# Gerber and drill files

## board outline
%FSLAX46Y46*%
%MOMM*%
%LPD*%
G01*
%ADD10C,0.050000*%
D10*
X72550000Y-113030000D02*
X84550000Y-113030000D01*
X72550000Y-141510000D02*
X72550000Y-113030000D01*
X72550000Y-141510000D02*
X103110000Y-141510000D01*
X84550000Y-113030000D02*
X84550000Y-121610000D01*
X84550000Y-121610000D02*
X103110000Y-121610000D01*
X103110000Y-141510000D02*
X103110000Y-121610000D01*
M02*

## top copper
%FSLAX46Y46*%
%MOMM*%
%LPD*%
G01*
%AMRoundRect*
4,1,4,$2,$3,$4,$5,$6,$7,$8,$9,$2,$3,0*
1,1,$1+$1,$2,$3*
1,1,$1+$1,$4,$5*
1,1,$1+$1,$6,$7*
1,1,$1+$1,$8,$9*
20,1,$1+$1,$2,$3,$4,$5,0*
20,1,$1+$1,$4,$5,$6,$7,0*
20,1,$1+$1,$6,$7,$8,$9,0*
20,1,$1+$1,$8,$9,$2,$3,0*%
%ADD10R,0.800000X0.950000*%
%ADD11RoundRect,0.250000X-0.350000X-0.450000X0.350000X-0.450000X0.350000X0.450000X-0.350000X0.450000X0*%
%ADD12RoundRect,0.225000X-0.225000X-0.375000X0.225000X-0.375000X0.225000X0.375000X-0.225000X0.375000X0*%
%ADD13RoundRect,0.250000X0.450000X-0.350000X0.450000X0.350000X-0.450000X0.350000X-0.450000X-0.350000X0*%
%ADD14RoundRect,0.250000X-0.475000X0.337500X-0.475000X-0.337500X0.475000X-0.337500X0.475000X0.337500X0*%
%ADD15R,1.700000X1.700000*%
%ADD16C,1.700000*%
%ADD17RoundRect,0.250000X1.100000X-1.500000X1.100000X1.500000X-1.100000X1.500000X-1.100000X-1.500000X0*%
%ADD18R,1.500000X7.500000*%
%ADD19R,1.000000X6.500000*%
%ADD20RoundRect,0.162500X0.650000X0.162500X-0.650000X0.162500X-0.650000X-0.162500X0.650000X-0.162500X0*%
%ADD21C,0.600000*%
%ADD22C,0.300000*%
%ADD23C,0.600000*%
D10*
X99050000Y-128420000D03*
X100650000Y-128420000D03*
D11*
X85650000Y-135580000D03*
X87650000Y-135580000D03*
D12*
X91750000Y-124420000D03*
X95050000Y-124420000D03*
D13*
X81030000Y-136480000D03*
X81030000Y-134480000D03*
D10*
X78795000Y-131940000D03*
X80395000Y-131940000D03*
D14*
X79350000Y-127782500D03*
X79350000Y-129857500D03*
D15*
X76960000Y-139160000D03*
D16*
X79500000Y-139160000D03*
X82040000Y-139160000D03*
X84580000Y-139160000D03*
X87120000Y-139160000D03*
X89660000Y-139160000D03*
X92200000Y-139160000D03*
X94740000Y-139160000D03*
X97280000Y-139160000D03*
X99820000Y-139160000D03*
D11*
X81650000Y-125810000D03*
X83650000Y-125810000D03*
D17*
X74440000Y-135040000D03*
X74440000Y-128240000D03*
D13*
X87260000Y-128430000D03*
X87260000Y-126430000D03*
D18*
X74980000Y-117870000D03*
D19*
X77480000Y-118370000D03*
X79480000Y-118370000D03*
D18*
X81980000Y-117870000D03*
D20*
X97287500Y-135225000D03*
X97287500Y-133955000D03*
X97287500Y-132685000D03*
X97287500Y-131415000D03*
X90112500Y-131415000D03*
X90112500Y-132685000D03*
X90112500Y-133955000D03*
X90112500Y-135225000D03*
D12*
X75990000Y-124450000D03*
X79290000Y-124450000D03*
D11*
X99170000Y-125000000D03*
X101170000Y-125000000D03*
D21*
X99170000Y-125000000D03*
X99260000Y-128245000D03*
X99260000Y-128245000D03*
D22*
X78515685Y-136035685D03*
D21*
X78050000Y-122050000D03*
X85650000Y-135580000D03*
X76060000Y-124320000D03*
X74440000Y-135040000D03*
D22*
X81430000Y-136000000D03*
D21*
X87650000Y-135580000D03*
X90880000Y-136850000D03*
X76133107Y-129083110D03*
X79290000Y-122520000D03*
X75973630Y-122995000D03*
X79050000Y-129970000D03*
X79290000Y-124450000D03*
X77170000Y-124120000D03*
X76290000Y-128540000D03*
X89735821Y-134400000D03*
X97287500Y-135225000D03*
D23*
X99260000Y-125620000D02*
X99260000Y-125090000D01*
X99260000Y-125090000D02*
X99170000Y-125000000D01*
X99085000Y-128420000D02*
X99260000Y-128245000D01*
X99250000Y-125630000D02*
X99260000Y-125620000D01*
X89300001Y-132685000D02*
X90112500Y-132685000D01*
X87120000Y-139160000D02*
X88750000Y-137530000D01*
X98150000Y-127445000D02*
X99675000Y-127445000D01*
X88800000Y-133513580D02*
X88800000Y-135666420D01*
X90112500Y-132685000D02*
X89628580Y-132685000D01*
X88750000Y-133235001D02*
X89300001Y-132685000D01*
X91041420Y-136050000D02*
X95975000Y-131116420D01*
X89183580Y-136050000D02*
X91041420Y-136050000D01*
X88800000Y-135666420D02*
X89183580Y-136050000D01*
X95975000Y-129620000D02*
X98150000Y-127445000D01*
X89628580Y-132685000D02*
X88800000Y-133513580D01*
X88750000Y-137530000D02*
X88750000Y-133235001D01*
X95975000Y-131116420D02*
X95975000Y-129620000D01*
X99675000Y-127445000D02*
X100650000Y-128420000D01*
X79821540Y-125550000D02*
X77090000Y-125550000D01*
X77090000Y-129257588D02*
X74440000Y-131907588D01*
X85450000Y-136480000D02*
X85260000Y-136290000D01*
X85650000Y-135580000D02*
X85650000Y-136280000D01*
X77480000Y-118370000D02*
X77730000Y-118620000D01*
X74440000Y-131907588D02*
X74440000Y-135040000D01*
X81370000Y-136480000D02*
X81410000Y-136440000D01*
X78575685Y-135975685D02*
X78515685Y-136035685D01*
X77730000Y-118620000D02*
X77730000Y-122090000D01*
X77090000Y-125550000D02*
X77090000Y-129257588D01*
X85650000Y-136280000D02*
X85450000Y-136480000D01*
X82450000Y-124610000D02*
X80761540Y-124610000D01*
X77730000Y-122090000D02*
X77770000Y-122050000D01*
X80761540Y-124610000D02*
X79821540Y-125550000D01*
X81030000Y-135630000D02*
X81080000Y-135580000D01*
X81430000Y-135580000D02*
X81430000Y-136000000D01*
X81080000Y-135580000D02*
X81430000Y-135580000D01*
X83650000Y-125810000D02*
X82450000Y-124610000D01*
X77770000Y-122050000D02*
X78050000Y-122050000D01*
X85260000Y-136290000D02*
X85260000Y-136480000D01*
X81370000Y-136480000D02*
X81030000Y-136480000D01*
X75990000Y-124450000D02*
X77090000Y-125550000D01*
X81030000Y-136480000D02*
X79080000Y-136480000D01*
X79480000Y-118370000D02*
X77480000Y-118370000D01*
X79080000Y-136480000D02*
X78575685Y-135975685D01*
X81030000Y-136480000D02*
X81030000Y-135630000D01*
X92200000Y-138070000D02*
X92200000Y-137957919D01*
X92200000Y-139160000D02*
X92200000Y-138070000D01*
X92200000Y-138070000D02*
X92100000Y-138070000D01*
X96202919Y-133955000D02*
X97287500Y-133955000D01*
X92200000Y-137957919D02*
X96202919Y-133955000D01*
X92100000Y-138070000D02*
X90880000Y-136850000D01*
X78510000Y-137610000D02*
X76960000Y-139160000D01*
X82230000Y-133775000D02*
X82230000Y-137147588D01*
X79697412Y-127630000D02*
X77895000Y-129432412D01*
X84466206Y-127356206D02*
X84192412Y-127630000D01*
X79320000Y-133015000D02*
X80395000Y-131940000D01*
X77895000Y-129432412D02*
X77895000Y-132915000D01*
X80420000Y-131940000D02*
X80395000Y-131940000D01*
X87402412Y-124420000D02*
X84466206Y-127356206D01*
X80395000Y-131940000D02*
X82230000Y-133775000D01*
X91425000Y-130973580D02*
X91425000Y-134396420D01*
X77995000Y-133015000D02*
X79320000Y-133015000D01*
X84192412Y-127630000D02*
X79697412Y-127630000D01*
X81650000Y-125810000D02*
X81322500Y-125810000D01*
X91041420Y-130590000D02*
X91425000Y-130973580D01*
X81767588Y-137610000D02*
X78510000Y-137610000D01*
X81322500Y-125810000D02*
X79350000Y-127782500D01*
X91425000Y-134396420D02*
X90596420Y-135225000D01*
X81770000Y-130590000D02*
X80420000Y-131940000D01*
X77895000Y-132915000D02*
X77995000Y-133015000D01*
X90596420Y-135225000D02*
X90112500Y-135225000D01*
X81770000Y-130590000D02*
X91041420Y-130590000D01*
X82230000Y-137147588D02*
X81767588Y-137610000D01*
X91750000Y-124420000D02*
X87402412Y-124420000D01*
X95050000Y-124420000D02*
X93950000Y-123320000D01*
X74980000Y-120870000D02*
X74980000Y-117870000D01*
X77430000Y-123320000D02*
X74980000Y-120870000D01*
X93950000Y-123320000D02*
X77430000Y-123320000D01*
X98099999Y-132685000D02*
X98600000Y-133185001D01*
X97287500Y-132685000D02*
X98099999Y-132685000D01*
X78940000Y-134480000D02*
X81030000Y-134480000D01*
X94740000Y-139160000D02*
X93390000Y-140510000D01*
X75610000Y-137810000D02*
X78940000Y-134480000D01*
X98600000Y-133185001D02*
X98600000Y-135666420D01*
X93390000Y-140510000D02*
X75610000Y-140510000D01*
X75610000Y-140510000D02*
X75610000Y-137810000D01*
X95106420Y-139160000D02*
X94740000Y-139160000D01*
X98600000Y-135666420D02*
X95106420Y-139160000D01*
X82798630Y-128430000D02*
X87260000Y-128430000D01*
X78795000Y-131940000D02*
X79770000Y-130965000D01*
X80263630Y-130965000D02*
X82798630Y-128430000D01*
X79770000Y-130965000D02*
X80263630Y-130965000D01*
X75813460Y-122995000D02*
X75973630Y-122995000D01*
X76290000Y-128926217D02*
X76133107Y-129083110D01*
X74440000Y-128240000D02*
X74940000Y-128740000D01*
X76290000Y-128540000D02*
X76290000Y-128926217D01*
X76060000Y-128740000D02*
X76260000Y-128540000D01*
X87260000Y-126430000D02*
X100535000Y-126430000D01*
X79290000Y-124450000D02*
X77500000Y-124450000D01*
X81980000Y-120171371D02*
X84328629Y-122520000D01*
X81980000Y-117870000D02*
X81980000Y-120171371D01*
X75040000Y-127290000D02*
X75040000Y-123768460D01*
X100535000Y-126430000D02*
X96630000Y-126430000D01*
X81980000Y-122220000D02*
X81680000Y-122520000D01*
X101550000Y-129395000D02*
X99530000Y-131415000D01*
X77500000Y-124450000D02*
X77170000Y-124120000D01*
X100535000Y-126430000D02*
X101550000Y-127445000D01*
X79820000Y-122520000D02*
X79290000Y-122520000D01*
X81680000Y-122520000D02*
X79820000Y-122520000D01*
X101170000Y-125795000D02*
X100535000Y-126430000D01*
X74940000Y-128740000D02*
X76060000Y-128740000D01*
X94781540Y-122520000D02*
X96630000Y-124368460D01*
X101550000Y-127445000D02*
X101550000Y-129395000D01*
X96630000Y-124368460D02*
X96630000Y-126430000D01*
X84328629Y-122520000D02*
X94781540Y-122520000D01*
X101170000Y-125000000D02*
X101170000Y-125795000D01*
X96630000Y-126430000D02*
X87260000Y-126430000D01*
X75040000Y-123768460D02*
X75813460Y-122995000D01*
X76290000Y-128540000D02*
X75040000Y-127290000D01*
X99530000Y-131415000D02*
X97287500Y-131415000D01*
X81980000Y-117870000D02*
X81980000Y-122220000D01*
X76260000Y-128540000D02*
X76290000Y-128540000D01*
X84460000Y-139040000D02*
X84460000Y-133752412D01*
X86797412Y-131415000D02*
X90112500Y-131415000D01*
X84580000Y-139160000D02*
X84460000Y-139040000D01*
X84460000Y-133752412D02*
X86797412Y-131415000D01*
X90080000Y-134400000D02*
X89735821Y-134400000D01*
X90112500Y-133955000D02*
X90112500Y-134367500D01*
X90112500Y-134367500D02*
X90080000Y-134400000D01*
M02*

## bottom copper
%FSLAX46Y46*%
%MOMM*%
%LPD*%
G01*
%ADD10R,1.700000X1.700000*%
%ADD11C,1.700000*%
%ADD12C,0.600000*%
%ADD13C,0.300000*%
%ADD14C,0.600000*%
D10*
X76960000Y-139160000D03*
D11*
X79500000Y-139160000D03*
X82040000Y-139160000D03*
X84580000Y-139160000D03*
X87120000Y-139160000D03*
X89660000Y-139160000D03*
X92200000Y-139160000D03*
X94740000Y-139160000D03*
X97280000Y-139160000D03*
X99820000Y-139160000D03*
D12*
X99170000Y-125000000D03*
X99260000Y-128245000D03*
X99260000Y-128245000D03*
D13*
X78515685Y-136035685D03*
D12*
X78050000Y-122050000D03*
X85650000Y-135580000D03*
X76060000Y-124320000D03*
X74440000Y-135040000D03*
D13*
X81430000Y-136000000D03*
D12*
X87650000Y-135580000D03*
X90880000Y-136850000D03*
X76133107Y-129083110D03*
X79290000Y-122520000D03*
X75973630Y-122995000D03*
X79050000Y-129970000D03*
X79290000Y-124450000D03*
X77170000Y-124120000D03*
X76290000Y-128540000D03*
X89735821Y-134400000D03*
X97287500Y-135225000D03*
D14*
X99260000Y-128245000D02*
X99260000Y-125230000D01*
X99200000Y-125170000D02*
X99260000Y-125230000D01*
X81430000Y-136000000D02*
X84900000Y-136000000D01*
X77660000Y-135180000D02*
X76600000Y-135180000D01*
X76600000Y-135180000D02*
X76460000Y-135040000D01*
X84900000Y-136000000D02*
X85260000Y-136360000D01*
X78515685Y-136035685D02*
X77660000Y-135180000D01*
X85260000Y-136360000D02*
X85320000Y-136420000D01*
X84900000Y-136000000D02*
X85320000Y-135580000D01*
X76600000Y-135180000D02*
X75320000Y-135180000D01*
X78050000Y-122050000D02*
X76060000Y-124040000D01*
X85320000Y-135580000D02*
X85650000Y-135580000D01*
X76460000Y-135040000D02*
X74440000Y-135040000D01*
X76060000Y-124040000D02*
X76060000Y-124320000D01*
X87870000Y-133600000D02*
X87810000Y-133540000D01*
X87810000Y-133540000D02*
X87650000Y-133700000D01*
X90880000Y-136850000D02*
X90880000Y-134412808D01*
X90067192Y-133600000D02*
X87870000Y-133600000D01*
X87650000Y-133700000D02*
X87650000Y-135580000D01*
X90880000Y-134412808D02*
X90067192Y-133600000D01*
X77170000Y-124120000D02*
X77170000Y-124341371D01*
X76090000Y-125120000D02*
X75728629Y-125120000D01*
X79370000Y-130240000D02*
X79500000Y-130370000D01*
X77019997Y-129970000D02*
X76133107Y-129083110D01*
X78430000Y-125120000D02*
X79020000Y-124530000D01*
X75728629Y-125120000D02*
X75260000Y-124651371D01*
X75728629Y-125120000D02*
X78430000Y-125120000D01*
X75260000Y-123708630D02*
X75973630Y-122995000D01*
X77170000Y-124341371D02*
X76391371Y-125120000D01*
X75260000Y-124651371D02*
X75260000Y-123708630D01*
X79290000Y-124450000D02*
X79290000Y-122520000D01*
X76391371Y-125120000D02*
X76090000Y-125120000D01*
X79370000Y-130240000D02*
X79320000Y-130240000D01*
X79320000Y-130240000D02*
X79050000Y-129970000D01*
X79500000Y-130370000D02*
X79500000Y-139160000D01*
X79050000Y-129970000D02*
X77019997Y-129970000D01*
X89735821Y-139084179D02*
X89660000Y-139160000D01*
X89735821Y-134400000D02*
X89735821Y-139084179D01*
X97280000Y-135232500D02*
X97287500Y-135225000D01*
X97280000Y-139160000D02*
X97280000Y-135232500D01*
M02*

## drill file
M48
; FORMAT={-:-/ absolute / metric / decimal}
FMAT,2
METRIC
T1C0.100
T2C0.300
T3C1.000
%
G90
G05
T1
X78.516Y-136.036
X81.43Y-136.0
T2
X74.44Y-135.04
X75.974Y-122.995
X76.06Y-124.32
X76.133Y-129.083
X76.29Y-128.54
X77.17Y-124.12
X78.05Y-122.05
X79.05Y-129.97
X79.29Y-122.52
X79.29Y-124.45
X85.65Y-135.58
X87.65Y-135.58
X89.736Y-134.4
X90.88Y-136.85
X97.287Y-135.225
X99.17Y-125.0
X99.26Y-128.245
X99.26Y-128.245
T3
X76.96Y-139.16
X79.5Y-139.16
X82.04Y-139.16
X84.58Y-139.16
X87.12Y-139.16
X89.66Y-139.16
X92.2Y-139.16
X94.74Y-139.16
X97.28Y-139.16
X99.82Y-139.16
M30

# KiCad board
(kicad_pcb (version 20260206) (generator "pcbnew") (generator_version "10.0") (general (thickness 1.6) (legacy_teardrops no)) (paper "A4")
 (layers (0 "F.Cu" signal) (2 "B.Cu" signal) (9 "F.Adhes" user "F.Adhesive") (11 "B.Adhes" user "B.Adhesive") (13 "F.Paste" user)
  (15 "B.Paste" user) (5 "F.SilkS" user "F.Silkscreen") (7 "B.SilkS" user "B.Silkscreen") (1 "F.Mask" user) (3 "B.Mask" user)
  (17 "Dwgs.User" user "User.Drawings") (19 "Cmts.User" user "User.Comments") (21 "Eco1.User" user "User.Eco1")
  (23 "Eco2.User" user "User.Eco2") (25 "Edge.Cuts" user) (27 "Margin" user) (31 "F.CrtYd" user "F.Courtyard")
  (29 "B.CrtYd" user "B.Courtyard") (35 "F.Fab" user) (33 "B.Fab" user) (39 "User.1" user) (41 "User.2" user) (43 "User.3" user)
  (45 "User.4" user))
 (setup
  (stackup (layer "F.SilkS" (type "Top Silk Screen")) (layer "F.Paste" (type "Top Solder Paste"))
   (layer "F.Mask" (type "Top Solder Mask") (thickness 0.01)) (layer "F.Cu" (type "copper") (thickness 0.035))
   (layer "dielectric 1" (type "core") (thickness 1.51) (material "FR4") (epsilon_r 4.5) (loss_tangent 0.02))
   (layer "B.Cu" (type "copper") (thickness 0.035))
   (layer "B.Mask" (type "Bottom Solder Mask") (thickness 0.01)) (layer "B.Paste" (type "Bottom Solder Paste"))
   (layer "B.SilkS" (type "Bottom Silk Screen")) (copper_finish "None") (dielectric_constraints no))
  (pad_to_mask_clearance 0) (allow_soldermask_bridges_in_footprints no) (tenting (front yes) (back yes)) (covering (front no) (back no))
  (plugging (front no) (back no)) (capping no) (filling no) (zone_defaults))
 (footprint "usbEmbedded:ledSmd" (layer "F.Cu") (at 99.85 128.97)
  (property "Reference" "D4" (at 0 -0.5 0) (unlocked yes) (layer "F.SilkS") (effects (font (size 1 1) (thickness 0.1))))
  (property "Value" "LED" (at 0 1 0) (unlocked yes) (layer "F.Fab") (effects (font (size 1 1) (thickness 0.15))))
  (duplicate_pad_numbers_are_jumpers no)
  (pad "1" smd rect (at -0.8 -0.55) (size 0.8 0.95) (layers "F.Cu" "F.Mask" "F.Paste") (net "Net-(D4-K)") (solder_mask_margin 0.1016))
  (pad "2" smd rect (at 0.8 -0.55) (size 0.8 0.95) (layers "F.Cu" "F.Mask" "F.Paste") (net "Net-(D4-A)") (solder_mask_margin 0.1016)))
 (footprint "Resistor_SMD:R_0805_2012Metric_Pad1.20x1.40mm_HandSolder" (layer "F.Cu") (at 86.65 135.58)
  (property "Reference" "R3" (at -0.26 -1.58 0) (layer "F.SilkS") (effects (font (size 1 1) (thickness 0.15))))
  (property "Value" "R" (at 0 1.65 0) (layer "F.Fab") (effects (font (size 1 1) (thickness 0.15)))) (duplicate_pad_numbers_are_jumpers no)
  (pad "1" smd roundrect (at -1 0) (size 1.2 1.4) (layers "F.Cu" "F.Mask" "F.Paste") (roundrect_rratio 0.208333) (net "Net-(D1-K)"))
  (pad "2" smd roundrect (at 1 0) (size 1.2 1.4) (layers "F.Cu" "F.Mask" "F.Paste") (roundrect_rratio 0.208333) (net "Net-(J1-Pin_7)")))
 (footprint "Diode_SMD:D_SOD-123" (layer "F.Cu") (at 93.4 124.42)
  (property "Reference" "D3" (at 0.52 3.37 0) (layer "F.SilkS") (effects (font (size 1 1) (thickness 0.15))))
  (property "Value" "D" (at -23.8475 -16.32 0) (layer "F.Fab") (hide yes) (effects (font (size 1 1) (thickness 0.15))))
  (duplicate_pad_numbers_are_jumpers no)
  (pad "1" smd roundrect (at -1.65 0) (size 0.9 1.2) (layers "F.Cu" "F.Mask" "F.Paste") (roundrect_rratio 0.25) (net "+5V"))
  (pad "2" smd roundrect (at 1.65 0) (size 0.9 1.2) (layers "F.Cu" "F.Mask" "F.Paste") (roundrect_rratio 0.25) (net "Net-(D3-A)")))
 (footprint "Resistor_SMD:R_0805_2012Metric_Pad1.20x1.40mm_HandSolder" (layer "F.Cu") (at 81.03 135.48 90)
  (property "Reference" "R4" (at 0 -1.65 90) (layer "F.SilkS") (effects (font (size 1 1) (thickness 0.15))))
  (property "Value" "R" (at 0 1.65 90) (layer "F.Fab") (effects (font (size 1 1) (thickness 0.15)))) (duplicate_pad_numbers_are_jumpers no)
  (pad "1" smd roundrect (at -1 0 90) (size 1.2 1.4) (layers "F.Cu" "F.Mask" "F.Paste") (roundrect_rratio 0.208333) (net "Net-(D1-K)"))
  (pad "2" smd roundrect (at 1 0 90) (size 1.2 1.4) (layers "F.Cu" "F.Mask" "F.Paste") (roundrect_rratio 0.208333) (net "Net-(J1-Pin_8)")))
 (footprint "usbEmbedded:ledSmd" (layer "F.Cu") (at 79.595 132.49)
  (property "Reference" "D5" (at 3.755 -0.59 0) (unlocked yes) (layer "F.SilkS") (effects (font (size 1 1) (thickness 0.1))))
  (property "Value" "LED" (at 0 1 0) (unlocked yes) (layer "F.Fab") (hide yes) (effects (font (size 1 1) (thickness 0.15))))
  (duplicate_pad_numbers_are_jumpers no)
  (pad "1" smd rect (at -0.8 -0.55) (size 0.8 0.95) (layers "F.Cu" "F.Mask" "F.Paste") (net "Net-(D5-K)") (solder_mask_margin 0.1016))
  (pad "2" smd rect (at 0.8 -0.55) (size 0.8 0.95) (layers "F.Cu" "F.Mask" "F.Paste") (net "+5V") (solder_mask_margin 0.1016)))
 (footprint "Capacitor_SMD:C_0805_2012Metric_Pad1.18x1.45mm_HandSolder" (layer "F.Cu") (at 79.35 128.82 -90)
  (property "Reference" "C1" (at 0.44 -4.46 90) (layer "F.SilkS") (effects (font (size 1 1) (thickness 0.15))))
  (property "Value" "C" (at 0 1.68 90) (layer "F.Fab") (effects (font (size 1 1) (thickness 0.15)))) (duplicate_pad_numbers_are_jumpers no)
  (pad "1" smd roundrect (at -1.0375 0 270) (size 1.175 1.45) (layers "F.Cu" "F.Mask" "F.Paste") (roundrect_rratio 0.212766) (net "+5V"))
  (pad "2" smd roundrect (at 1.0375 0 270) (size 1.175 1.45) (layers "F.Cu" "F.Mask" "F.Paste") (roundrect_rratio 0.212766) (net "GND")))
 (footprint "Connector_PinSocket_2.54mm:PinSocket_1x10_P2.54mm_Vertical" (layer "F.Cu") (at 76.96 139.16 90)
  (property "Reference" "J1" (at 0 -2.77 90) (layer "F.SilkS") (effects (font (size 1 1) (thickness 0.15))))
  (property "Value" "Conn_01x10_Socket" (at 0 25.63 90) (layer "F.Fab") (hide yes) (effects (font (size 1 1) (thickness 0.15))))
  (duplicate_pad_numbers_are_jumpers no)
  (pad "1" thru_hole rect (at 0 0 90) (size 1.7 1.7) (drill 1) (layers "*.Cu" "*.Mask") (remove_unused_layers no) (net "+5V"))
  (pad "2" thru_hole circle (at 0 2.54 90) (size 1.7 1.7) (drill 1) (layers "*.Cu" "*.Mask") (remove_unused_layers no) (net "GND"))
  (pad "3" thru_hole circle (at 0 5.08 90) (size 1.7 1.7) (drill 1) (layers "*.Cu" "*.Mask") (remove_unused_layers no)
   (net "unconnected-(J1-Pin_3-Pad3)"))
  (pad "4" thru_hole circle (at 0 7.62 90) (size 1.7 1.7) (drill 1) (layers "*.Cu" "*.Mask") (remove_unused_layers no)
   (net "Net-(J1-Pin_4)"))
  (pad "5" thru_hole circle (at 0 10.16 90) (size 1.7 1.7) (drill 1) (layers "*.Cu" "*.Mask") (remove_unused_layers no) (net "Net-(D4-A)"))
  (pad "6" thru_hole circle (at 0 12.7 90) (size 1.7 1.7) (drill 1) (layers "*.Cu" "*.Mask") (remove_unused_layers no)
   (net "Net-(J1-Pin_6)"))
  (pad "7" thru_hole circle (at 0 15.24 90) (size 1.7 1.7) (drill 1) (layers "*.Cu" "*.Mask") (remove_unused_layers no)
   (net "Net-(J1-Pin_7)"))
  (pad "8" thru_hole circle (at 0 17.78 90) (size 1.7 1.7) (drill 1) (layers "*.Cu" "*.Mask") (remove_unused_layers no)
   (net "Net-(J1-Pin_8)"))
  (pad "9" thru_hole circle (at 0 20.32 90) (size 1.7 1.7) (drill 1) (layers "*.Cu" "*.Mask") (remove_unused_layers no)
   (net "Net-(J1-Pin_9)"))
  (pad "10" thru_hole circle (at 0 22.86 90) (size 1.7 1.7) (drill 1) (layers "*.Cu" "*.Mask") (remove_unused_layers no)
   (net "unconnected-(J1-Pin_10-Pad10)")))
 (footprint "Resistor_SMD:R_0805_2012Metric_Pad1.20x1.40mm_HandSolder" (layer "F.Cu") (at 82.65 125.81)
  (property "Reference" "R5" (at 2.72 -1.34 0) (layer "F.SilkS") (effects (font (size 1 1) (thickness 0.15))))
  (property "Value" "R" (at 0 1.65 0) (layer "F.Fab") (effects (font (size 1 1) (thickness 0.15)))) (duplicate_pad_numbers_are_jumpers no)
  (pad "1" smd roundrect (at -1 0) (size 1.2 1.4) (layers "F.Cu" "F.Mask" "F.Paste") (roundrect_rratio 0.208333) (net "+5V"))
  (pad "2" smd roundrect (at 1 0) (size 1.2 1.4) (layers "F.Cu" "F.Mask" "F.Paste") (roundrect_rratio 0.208333) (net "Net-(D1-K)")))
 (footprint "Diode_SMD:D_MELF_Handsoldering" (layer "F.Cu") (at 74.44 131.64 90)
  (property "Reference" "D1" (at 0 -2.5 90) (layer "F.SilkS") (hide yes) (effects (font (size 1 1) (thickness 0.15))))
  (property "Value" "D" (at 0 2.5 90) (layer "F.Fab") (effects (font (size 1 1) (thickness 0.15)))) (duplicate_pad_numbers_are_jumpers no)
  (pad "1" smd roundrect (at -3.4 0 90) (size 3.5 2.7) (layers "F.Cu" "F.Mask" "F.Paste") (roundrect_rratio 0.0925925926) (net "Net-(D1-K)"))
  (pad "2" smd roundrect (at 3.4 0 90) (size 3.5 2.7) (layers "F.Cu" "F.Mask" "F.Paste") (roundrect_rratio 0.0925925926) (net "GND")))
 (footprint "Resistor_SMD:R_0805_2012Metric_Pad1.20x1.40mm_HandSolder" (layer "F.Cu") (at 87.26 127.43 90)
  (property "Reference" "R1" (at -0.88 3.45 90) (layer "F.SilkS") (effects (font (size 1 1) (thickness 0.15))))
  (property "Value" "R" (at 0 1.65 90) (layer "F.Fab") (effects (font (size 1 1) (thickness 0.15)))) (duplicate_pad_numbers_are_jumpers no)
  (pad "1" smd roundrect (at -1 0 90) (size 1.2 1.4) (layers "F.Cu" "F.Mask" "F.Paste") (roundrect_rratio 0.208333) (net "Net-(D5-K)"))
  (pad "2" smd roundrect (at 1 0 90) (size 1.2 1.4) (layers "F.Cu" "F.Mask" "F.Paste") (roundrect_rratio 0.208333) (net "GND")))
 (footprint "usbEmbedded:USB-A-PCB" (layer "F.Cu") (at 78.48 118.07 -90)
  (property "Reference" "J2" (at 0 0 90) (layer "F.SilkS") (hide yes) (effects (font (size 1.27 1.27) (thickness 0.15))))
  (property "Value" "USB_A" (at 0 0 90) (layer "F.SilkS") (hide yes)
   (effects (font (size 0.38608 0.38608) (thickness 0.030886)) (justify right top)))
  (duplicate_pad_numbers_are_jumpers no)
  (pad "1" smd rect (at -0.2 3.5 270) (size 7.5 1.5) (layers "F.Cu" "F.Mask" "F.Paste") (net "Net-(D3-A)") (solder_mask_margin 0.1016))
  (pad "2" smd rect (at 0.3 1 270) (size 6.5 1) (layers "F.Cu" "F.Mask" "F.Paste") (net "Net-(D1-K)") (solder_mask_margin 0.1016))
  (pad "3" smd rect (at 0.3 -1 270) (size 6.5 1) (layers "F.Cu" "F.Mask" "F.Paste") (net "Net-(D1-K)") (solder_mask_margin 0.1016))
  (pad "4" smd rect (at -0.2 -3.5 270) (size 7.5 1.5) (layers "F.Cu" "F.Mask" "F.Paste") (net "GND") (solder_mask_margin 0.1016)))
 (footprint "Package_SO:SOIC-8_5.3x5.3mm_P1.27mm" (layer "F.Cu") (at 93.7 133.32 180)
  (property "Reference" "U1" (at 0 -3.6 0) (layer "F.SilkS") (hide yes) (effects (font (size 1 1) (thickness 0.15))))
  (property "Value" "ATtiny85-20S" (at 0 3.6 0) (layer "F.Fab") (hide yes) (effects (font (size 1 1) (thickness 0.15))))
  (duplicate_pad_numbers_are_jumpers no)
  (pad "1" smd roundrect (at -3.5875 -1.905 180) (size 1.625 0.65) (layers "F.Cu" "F.Mask" "F.Paste") (roundrect_rratio 0.25)
   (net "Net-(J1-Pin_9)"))
  (pad "2" smd roundrect (at -3.5875 -0.635 180) (size 1.625 0.65) (layers "F.Cu" "F.Mask" "F.Paste") (roundrect_rratio 0.25)
   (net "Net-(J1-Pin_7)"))
  (pad "3" smd roundrect (at -3.5875 0.635 180) (size 1.625 0.65) (layers "F.Cu" "F.Mask" "F.Paste") (roundrect_rratio 0.25)
   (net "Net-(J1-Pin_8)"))
  (pad "4" smd roundrect (at -3.5875 1.905 180) (size 1.625 0.65) (layers "F.Cu" "F.Mask" "F.Paste") (roundrect_rratio 0.25) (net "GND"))
  (pad "5" smd roundrect (at 3.5875 1.905 180) (size 1.625 0.65) (layers "F.Cu" "F.Mask" "F.Paste") (roundrect_rratio 0.25)
   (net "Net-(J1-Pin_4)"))
  (pad "6" smd roundrect (at 3.5875 0.635 180) (size 1.625 0.65) (layers "F.Cu" "F.Mask" "F.Paste") (roundrect_rratio 0.25)
   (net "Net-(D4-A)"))
  (pad "7" smd roundrect (at 3.5875 -0.635 180) (size 1.625 0.65) (layers "F.Cu" "F.Mask" "F.Paste") (roundrect_rratio 0.25)
   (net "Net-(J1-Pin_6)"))
  (pad "8" smd roundrect (at 3.5875 -1.905 180) (size 1.625 0.65) (layers "F.Cu" "F.Mask" "F.Paste") (roundrect_rratio 0.25) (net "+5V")))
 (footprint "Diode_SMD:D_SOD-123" (layer "F.Cu") (at 77.64 124.45)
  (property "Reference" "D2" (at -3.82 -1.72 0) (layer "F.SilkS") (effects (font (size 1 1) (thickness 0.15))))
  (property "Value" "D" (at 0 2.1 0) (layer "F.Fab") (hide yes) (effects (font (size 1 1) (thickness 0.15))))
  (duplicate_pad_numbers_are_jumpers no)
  (pad "1" smd roundrect (at -1.65 0) (size 0.9 1.2) (layers "F.Cu" "F.Mask" "F.Paste") (roundrect_rratio 0.25) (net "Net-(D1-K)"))
  (pad "2" smd roundrect (at 1.65 0) (size 0.9 1.2) (layers "F.Cu" "F.Mask" "F.Paste") (roundrect_rratio 0.25) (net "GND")))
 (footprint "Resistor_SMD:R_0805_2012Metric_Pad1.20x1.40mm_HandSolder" (layer "F.Cu") (at 100.17 125)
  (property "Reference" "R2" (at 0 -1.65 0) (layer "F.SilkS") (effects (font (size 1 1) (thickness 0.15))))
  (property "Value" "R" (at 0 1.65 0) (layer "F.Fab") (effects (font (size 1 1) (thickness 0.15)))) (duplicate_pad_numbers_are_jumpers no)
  (pad "1" smd roundrect (at -1 0) (size 1.2 1.4) (layers "F.Cu" "F.Mask" "F.Paste") (roundrect_rratio 0.208333) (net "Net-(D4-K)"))
  (pad "2" smd roundrect (at 1 0) (size 1.2 1.4) (layers "F.Cu" "F.Mask" "F.Paste") (roundrect_rratio 0.208333) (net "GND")))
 (gr_line (start 72.55 113.03) (end 84.55 113.03) (stroke (width 0.05) (type solid)) (layer "Edge.Cuts"))
 (gr_line (start 72.55 141.51) (end 72.55 113.03) (stroke (width 0.05) (type solid)) (layer "Edge.Cuts"))
 (gr_line (start 72.55 141.51) (end 103.11 141.51) (stroke (width 0.05) (type default)) (layer "Edge.Cuts"))
 (gr_line (start 84.55 113.03) (end 84.55 121.61) (stroke (width 0.05) (type solid)) (layer "Edge.Cuts"))
 (gr_line (start 84.55 121.61) (end 103.11 121.61) (stroke (width 0.05) (type default)) (layer "Edge.Cuts"))
 (gr_line (start 103.11 141.51) (end 103.11 121.61) (stroke (width 0.05) (type solid)) (layer "Edge.Cuts"))
 (segment (start 99.26 125.62) (end 99.26 125.09) (width 0.6) (layer "F.Cu") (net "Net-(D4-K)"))
 (segment (start 99.26 125.09) (end 99.17 125) (width 0.6) (layer "F.Cu") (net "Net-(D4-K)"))
 (segment (start 99.085 128.42) (end 99.26 128.245) (width 0.6) (layer "F.Cu") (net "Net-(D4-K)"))
 (segment (start 99.25 125.63) (end 99.26 125.62) (width 0.6) (layer "F.Cu") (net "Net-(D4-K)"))
 (via (at 99.17 125) (size 0.6) (drill 0.3) (layers "F.Cu" "B.Cu") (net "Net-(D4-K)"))
 (via (at 99.26 128.245) (size 0.6) (drill 0.3) (layers "F.Cu" "B.Cu") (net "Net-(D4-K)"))
 (via (at 99.26 128.245) (size 0.6) (drill 0.3) (layers "F.Cu" "B.Cu") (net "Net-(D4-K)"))
 (segment (start 99.26 128.245) (end 99.26 125.23) (width 0.6) (layer "B.Cu") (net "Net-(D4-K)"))
 (segment (start 99.2 125.17) (end 99.26 125.23) (width 0.6) (layer "B.Cu") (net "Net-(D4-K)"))
 (segment (start 89.300001 132.685) (end 90.1125 132.685) (width 0.6) (layer "F.Cu") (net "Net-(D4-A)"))
 (segment (start 87.12 139.16) (end 88.75 137.53) (width 0.6) (layer "F.Cu") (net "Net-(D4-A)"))
 (segment (start 98.15 127.445) (end 99.675 127.445) (width 0.6) (layer "F.Cu") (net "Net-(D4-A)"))
 (segment (start 88.8 133.51358) (end 88.8 135.66642) (width 0.6) (layer "F.Cu") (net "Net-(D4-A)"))
 (segment (start 90.1125 132.685) (end 89.62858 132.685) (width 0.6) (layer "F.Cu") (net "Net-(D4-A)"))
 (segment (start 88.75 133.235001) (end 89.300001 132.685) (width 0.6) (layer "F.Cu") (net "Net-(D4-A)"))
 (segment (start 91.04142 136.05) (end 95.975 131.11642) (width 0.6) (layer "F.Cu") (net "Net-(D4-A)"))
 (segment (start 89.18358 136.05) (end 91.04142 136.05) (width 0.6) (layer "F.Cu") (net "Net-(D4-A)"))
 (segment (start 88.8 135.66642) (end 89.18358 136.05) (width 0.6) (layer "F.Cu") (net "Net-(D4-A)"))
 (segment (start 95.975 129.62) (end 98.15 127.445) (width 0.6) (layer "F.Cu") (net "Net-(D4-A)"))
 (segment (start 89.62858 132.685) (end 88.8 133.51358) (width 0.6) (layer "F.Cu") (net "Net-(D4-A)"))
 (segment (start 88.75 137.53) (end 88.75 133.235001) (width 0.6) (layer "F.Cu") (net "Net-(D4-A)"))
 (segment (start 95.975 131.11642) (end 95.975 129.62) (width 0.6) (layer "F.Cu") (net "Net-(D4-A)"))
 (segment (start 99.675 127.445) (end 100.65 128.42) (width 0.6) (layer "F.Cu") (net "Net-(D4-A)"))
 (segment (start 79.82154 125.55) (end 77.09 125.55) (width 0.6) (layer "F.Cu") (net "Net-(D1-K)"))
 (segment (start 77.09 129.257588) (end 74.44 131.907588) (width 0.6) (layer "F.Cu") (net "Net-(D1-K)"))
 (segment (start 85.45 136.48) (end 85.26 136.29) (width 0.6) (layer "F.Cu") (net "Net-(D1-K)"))
 (segment (start 85.65 135.58) (end 85.65 136.28) (width 0.6) (layer "F.Cu") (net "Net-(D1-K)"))
 (segment (start 77.48 118.37) (end 77.73 118.62) (width 0.6) (layer "F.Cu") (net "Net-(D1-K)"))
 (segment (start 74.44 131.907588) (end 74.44 135.04) (width 0.6) (layer "F.Cu") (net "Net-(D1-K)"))
 (segment (start 81.37 136.48) (end 81.41 136.44) (width 0.6) (layer "F.Cu") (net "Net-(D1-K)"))
 (segment (start 78.575685 135.975685) (end 78.515685 136.035685) (width 0.6) (layer "F.Cu") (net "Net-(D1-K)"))
 (segment (start 77.73 118.62) (end 77.73 122.09) (width 0.6) (layer "F.Cu") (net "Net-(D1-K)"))
 (segment (start 77.09 125.55) (end 77.09 129.257588) (width 0.6) (layer "F.Cu") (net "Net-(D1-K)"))
 (segment (start 85.65 136.28) (end 85.45 136.48) (width 0.6) (layer "F.Cu") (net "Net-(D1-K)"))
 (segment (start 82.45 124.61) (end 80.76154 124.61) (width 0.6) (layer "F.Cu") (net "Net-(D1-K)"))
 (segment (start 77.73 122.09) (end 77.77 122.05) (width 0.6) (layer "F.Cu") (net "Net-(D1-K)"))
 (segment (start 80.76154 124.61) (end 79.82154 125.55) (width 0.6) (layer "F.Cu") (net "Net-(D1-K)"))
 (segment (start 81.03 135.63) (end 81.08 135.58) (width 0.6) (layer "F.Cu") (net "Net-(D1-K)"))
 (segment (start 81.43 135.58) (end 81.43 136) (width 0.6) (layer "F.Cu") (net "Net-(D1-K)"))
 (segment (start 81.08 135.58) (end 81.43 135.58) (width 0.6) (layer "F.Cu") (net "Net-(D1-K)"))
 (segment (start 83.65 125.81) (end 82.45 124.61) (width 0.6) (layer "F.Cu") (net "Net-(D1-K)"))
 (segment (start 77.77 122.05) (end 78.05 122.05) (width 0.6) (layer "F.Cu") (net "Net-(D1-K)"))
 (segment (start 85.26 136.29) (end 85.26 136.48) (width 0.6) (layer "F.Cu") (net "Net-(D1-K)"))
 (segment (start 81.37 136.48) (end 81.03 136.48) (width 0.6) (layer "F.Cu") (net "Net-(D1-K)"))
 (segment (start 75.99 124.45) (end 77.09 125.55) (width 0.6) (layer "F.Cu") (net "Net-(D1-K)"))
 (segment (start 81.03 136.48) (end 79.08 136.48) (width 0.6) (layer "F.Cu") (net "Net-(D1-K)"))
 (segment (start 79.48 118.37) (end 77.48 118.37) (width 0.6) (layer "F.Cu") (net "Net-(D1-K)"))
 (segment (start 79.08 136.48) (end 78.575685 135.975685) (width 0.6) (layer "F.Cu") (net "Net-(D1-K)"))
 (segment (start 81.03 136.48) (end 81.03 135.63) (width 0.6) (layer "F.Cu") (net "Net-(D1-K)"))
 (via micro (at 78.515685 136.035685) (size 0.3) (drill 0.1) (layers "F.Cu" "B.Cu") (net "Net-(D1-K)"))
 (via (at 78.05 122.05) (size 0.6) (drill 0.3) (layers "F.Cu" "B.Cu") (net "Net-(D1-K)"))
 (via (at 85.65 135.58) (size 0.6) (drill 0.3) (layers "F.Cu" "B.Cu") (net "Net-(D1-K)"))
 (via (at 76.06 124.32) (size 0.6) (drill 0.3) (layers "F.Cu" "B.Cu") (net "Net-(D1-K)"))
 (via (at 74.44 135.04) (size 0.6) (drill 0.3) (layers "F.Cu" "B.Cu") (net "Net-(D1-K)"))
 (via micro (at 81.43 136) (size 0.3) (drill 0.1) (layers "F.Cu" "B.Cu") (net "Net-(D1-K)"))
 (segment (start 81.43 136) (end 84.9 136) (width 0.6) (layer "B.Cu") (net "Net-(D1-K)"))
 (segment (start 77.66 135.18) (end 76.6 135.18) (width 0.6) (layer "B.Cu") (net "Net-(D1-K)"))
 (segment (start 76.6 135.18) (end 76.46 135.04) (width 0.6) (layer "B.Cu") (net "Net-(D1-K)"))
 (segment (start 84.9 136) (end 85.26 136.36) (width 0.6) (layer "B.Cu") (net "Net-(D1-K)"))
 (segment (start 78.515685 136.035685) (end 77.66 135.18) (width 0.6) (layer "B.Cu") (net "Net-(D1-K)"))
 (segment (start 85.26 136.36) (end 85.32 136.42) (width 0.6) (layer "B.Cu") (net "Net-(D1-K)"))
 (segment (start 84.9 136) (end 85.32 135.58) (width 0.6) (layer "B.Cu") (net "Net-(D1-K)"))
 (segment (start 76.6 135.18) (end 75.32 135.18) (width 0.6) (layer "B.Cu") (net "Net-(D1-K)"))
 (segment (start 78.05 122.05) (end 76.06 124.04) (width 0.6) (layer "B.Cu") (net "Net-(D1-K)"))
 (segment (start 85.32 135.58) (end 85.65 135.58) (width 0.6) (layer "B.Cu") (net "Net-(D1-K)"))
 (segment (start 76.46 135.04) (end 74.44 135.04) (width 0.6) (layer "B.Cu") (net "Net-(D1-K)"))
 (segment (start 76.06 124.04) (end 76.06 124.32) (width 0.6) (layer "B.Cu") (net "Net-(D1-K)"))
 (segment (start 92.2 138.07) (end 92.2 137.957919) (width 0.6) (layer "F.Cu") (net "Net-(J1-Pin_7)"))
 (segment (start 92.2 139.16) (end 92.2 138.07) (width 0.6) (layer "F.Cu") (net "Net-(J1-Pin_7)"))
 (segment (start 92.2 138.07) (end 92.1 138.07) (width 0.6) (layer "F.Cu") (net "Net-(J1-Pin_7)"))
 (segment (start 96.202919 133.955) (end 97.2875 133.955) (width 0.6) (layer "F.Cu") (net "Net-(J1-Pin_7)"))
 (segment (start 92.2 137.957919) (end 96.202919 133.955) (width 0.6) (layer "F.Cu") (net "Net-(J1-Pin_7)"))
 (segment (start 92.1 138.07) (end 90.88 136.85) (width 0.6) (layer "F.Cu") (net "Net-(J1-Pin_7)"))
 (via (at 87.65 135.58) (size 0.6) (drill 0.3) (layers "F.Cu" "B.Cu") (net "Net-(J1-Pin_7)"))
 (via (at 90.88 136.85) (size 0.6) (drill 0.3) (layers "F.Cu" "B.Cu") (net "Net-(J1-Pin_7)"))
 (segment (start 87.87 133.6) (end 87.81 133.54) (width 0.6) (layer "B.Cu") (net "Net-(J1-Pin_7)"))
 (segment (start 87.81 133.54) (end 87.65 133.7) (width 0.6) (layer "B.Cu") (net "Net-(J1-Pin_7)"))
 (segment (start 90.88 136.85) (end 90.88 134.412808) (width 0.6) (layer "B.Cu") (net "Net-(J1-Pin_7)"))
 (segment (start 90.067192 133.6) (end 87.87 133.6) (width 0.6) (layer "B.Cu") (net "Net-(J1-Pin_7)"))
 (segment (start 87.65 133.7) (end 87.65 135.58) (width 0.6) (layer "B.Cu") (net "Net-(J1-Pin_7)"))
 (segment (start 90.88 134.412808) (end 90.067192 133.6) (width 0.6) (layer "B.Cu") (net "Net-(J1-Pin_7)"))
 (segment (start 78.51 137.61) (end 76.96 139.16) (width 0.6) (layer "F.Cu") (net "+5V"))
 (segment (start 82.23 133.775) (end 82.23 137.147588) (width 0.6) (layer "F.Cu") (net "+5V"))
 (segment (start 79.697412 127.63) (end 77.895 129.432412) (width 0.6) (layer "F.Cu") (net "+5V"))
 (segment (start 84.466206 127.356206) (end 84.192412 127.63) (width 0.6) (layer "F.Cu") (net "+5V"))
 (segment (start 79.32 133.015) (end 80.395 131.94) (width 0.6) (layer "F.Cu") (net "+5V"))
 (segment (start 77.895 129.432412) (end 77.895 132.915) (width 0.6) (layer "F.Cu") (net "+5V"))
 (segment (start 80.42 131.94) (end 80.395 131.94) (width 0.6) (layer "F.Cu") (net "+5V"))
 (segment (start 87.402412 124.42) (end 84.466206 127.356206) (width 0.6) (layer "F.Cu") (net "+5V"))
 (segment (start 80.395 131.94) (end 82.23 133.775) (width 0.6) (layer "F.Cu") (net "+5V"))
 (segment (start 91.425 130.97358) (end 91.425 134.39642) (width 0.6) (layer "F.Cu") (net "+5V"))
 (segment (start 77.995 133.015) (end 79.32 133.015) (width 0.6) (layer "F.Cu") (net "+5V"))
 (segment (start 84.192412 127.63) (end 79.697412 127.63) (width 0.6) (layer "F.Cu") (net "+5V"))
 (segment (start 81.65 125.81) (end 81.3225 125.81) (width 0.6) (layer "F.Cu") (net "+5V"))
 (segment (start 91.04142 130.59) (end 91.425 130.97358) (width 0.6) (layer "F.Cu") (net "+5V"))
 (segment (start 81.767588 137.61) (end 78.51 137.61) (width 0.6) (layer "F.Cu") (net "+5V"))
 (segment (start 81.3225 125.81) (end 79.35 127.7825) (width 0.6) (layer "F.Cu") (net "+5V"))
 (segment (start 91.425 134.39642) (end 90.59642 135.225) (width 0.6) (layer "F.Cu") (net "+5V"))
 (segment (start 81.77 130.59) (end 80.42 131.94) (width 0.6) (layer "F.Cu") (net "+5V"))
 (segment (start 77.895 132.915) (end 77.995 133.015) (width 0.6) (layer "F.Cu") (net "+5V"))
 (segment (start 90.59642 135.225) (end 90.1125 135.225) (width 0.6) (layer "F.Cu") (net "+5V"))
 (segment (start 81.77 130.59) (end 91.04142 130.59) (width 0.6) (layer "F.Cu") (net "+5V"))
 (segment (start 82.23 137.147588) (end 81.767588 137.61) (width 0.6) (layer "F.Cu") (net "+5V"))
 (segment (start 91.75 124.42) (end 87.402412 124.42) (width 0.6) (layer "F.Cu") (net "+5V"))
 (segment (start 95.05 124.42) (end 93.95 123.32) (width 0.6) (layer "F.Cu") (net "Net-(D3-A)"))
 (segment (start 74.98 120.87) (end 74.98 117.87) (width 0.6) (layer "F.Cu") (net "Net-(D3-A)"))
 (segment (start 77.43 123.32) (end 74.98 120.87) (width 0.6) (layer "F.Cu") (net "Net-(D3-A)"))
 (segment (start 93.95 123.32) (end 77.43 123.32) (width 0.6) (layer "F.Cu") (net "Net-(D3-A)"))
 (segment (start 98.099999 132.685) (end 98.6 133.185001) (width 0.6) (layer "F.Cu") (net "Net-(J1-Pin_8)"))
 (segment (start 97.2875 132.685) (end 98.099999 132.685) (width 0.6) (layer "F.Cu") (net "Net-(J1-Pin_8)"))
 (segment (start 78.94 134.48) (end 81.03 134.48) (width 0.6) (layer "F.Cu") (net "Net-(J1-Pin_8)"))
 (segment (start 94.74 139.16) (end 93.39 140.51) (width 0.6) (layer "F.Cu") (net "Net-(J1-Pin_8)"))
 (segment (start 75.61 137.81) (end 78.94 134.48) (width 0.6) (layer "F.Cu") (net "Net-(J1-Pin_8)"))
 (segment (start 98.6 133.185001) (end 98.6 135.66642) (width 0.6) (layer "F.Cu") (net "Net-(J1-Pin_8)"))
 (segment (start 93.39 140.51) (end 75.61 140.51) (width 0.6) (layer "F.Cu") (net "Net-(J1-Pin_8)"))
 (segment (start 75.61 140.51) (end 75.61 137.81) (width 0.6) (layer "F.Cu") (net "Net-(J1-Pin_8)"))
 (segment (start 95.10642 139.16) (end 94.74 139.16) (width 0.6) (layer "F.Cu") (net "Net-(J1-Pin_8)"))
 (segment (start 98.6 135.66642) (end 95.10642 139.16) (width 0.6) (layer "F.Cu") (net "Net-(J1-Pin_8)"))
 (segment (start 82.79863 128.43) (end 87.26 128.43) (width 0.6) (layer "F.Cu") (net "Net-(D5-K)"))
 (segment (start 78.795 131.94) (end 79.77 130.965) (width 0.6) (layer "F.Cu") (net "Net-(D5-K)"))
 (segment (start 80.26363 130.965) (end 82.79863 128.43) (width 0.6) (layer "F.Cu") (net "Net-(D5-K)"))
 (segment (start 79.77 130.965) (end 80.26363 130.965) (width 0.6) (layer "F.Cu") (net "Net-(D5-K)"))
 (segment (start 75.81346 122.995) (end 75.97363 122.995) (width 0.6) (layer "F.Cu") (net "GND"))
 (segment (start 76.29 128.926217) (end 76.133107 129.08311) (width 0.6) (layer "F.Cu") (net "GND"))
 (segment (start 74.44 128.24) (end 74.94 128.74) (width 0.6) (layer "F.Cu") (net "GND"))
 (segment (start 76.29 128.54) (end 76.29 128.926217) (width 0.6) (layer "F.Cu") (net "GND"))
 (segment (start 76.06 128.74) (end 76.26 128.54) (width 0.6) (layer "F.Cu") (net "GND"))
 (segment (start 87.26 126.43) (end 100.535 126.43) (width 0.6) (layer "F.Cu") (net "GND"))
 (segment (start 79.29 124.45) (end 77.5 124.45) (width 0.6) (layer "F.Cu") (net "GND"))
 (segment (start 81.98 120.171371) (end 84.328629 122.52) (width 0.6) (layer "F.Cu") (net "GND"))
 (segment (start 81.98 117.87) (end 81.98 120.171371) (width 0.6) (layer "F.Cu") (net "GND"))
 (segment (start 75.04 127.29) (end 75.04 123.76846) (width 0.6) (layer "F.Cu") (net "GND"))
 (segment (start 100.535 126.43) (end 96.63 126.43) (width 0.6) (layer "F.Cu") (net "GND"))
 (segment (start 81.98 122.22) (end 81.68 122.52) (width 0.6) (layer "F.Cu") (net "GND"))
 (segment (start 101.55 129.395) (end 99.53 131.415) (width 0.6) (layer "F.Cu") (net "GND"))
 (segment (start 77.5 124.45) (end 77.17 124.12) (width 0.6) (layer "F.Cu") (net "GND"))
 (segment (start 100.535 126.43) (end 101.55 127.445) (width 0.6) (layer "F.Cu") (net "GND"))
 (segment (start 79.82 122.52) (end 79.29 122.52) (width 0.6) (layer "F.Cu") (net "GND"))
 (segment (start 81.68 122.52) (end 79.82 122.52) (width 0.6) (layer "F.Cu") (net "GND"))
 (segment (start 101.17 125.795) (end 100.535 126.43) (width 0.6) (layer "F.Cu") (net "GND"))
 (segment (start 74.94 128.74) (end 76.06 128.74) (width 0.6) (layer "F.Cu") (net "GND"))
 (segment (start 94.78154 122.52) (end 96.63 124.36846) (width 0.6) (layer "F.Cu") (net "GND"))
 (segment (start 101.55 127.445) (end 101.55 129.395) (width 0.6) (layer "F.Cu") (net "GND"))
 (segment (start 96.63 124.36846) (end 96.63 126.43) (width 0.6) (layer "F.Cu") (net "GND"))
 (segment (start 84.328629 122.52) (end 94.78154 122.52) (width 0.6) (layer "F.Cu") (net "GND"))
 (segment (start 101.17 125) (end 101.17 125.795) (width 0.6) (layer "F.Cu") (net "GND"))
 (segment (start 96.63 126.43) (end 87.26 126.43) (width 0.6) (layer "F.Cu") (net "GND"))
 (segment (start 75.04 123.76846) (end 75.81346 122.995) (width 0.6) (layer "F.Cu") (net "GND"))
 (segment (start 76.29 128.54) (end 75.04 127.29) (width 0.6) (layer "F.Cu") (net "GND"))
 (segment (start 99.53 131.415) (end 97.2875 131.415) (width 0.6) (layer "F.Cu") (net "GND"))
 (segment (start 81.98 117.87) (end 81.98 122.22) (width 0.6) (layer "F.Cu") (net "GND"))
 (segment (start 76.26 128.54) (end 76.29 128.54) (width 0.6) (layer "F.Cu") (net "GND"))
 (via (at 76.133107 129.08311) (size 0.6) (drill 0.3) (layers "F.Cu" "B.Cu") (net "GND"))
 (via (at 79.29 122.52) (size 0.6) (drill 0.3) (layers "F.Cu" "B.Cu") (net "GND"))
 (via (at 75.97363 122.995) (size 0.6) (drill 0.3) (layers "F.Cu" "B.Cu") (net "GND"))
 (via (at 79.05 129.97) (size 0.6) (drill 0.3) (layers "F.Cu" "B.Cu") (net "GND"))
 (via (at 79.29 124.45) (size 0.6) (drill 0.3) (layers "F.Cu" "B.Cu") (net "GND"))
 (via (at 77.17 124.12) (size 0.6) (drill 0.3) (layers "F.Cu" "B.Cu") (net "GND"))
 (via (at 76.29 128.54) (size 0.6) (drill 0.3) (layers "F.Cu" "B.Cu") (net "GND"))
 (segment (start 77.17 124.12) (end 77.17 124.341371) (width 0.6) (layer "B.Cu") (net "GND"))
 (segment (start 76.09 125.12) (end 75.728629 125.12) (width 0.6) (layer "B.Cu") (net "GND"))
 (segment (start 79.37 130.24) (end 79.5 130.37) (width 0.6) (layer "B.Cu") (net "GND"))
 (segment (start 77.019997 129.97) (end 76.133107 129.08311) (width 0.6) (layer "B.Cu") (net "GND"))
 (segment (start 78.43 125.12) (end 79.02 124.53) (width 0.6) (layer "B.Cu") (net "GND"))
 (segment (start 75.728629 125.12) (end 75.26 124.651371) (width 0.6) (layer "B.Cu") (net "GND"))
 (segment (start 75.728629 125.12) (end 78.43 125.12) (width 0.6) (layer "B.Cu") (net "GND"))
 (segment (start 75.26 123.70863) (end 75.97363 122.995) (width 0.6) (layer "B.Cu") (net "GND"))
 (segment (start 77.17 124.341371) (end 76.391371 125.12) (width 0.6) (layer "B.Cu") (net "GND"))
 (segment (start 75.26 124.651371) (end 75.26 123.70863) (width 0.6) (layer "B.Cu") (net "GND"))
 (segment (start 79.29 124.45) (end 79.29 122.52) (width 0.6) (layer "B.Cu") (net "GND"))
 (segment (start 76.391371 125.12) (end 76.09 125.12) (width 0.6) (layer "B.Cu") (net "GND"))
 (segment (start 79.37 130.24) (end 79.32 130.24) (width 0.6) (layer "B.Cu") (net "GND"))
 (segment (start 79.32 130.24) (end 79.05 129.97) (width 0.6) (layer "B.Cu") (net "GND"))
 (segment (start 79.5 130.37) (end 79.5 139.16) (width 0.6) (layer "B.Cu") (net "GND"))
 (segment (start 79.05 129.97) (end 77.019997 129.97) (width 0.6) (layer "B.Cu") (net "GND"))
 (segment (start 84.46 139.04) (end 84.46 133.752412) (width 0.6) (layer "F.Cu") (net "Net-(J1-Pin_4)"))
 (segment (start 86.797412 131.415) (end 90.1125 131.415) (width 0.6) (layer "F.Cu") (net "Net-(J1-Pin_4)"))
 (segment (start 84.58 139.16) (end 84.46 139.04) (width 0.6) (layer "F.Cu") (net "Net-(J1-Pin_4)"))
 (segment (start 84.46 133.752412) (end 86.797412 131.415) (width 0.6) (layer "F.Cu") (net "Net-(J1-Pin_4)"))
 (segment (start 90.08 134.4) (end 89.735821 134.4) (width 0.6) (layer "F.Cu") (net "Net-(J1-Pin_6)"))
 (segment (start 90.1125 133.955) (end 90.1125 134.3675) (width 0.6) (layer "F.Cu") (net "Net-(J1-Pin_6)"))
 (segment (start 90.1125 134.3675) (end 90.08 134.4) (width 0.6) (layer "F.Cu") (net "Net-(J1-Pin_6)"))
 (via (at 89.735821 134.4) (size 0.6) (drill 0.3) (layers "F.Cu" "B.Cu") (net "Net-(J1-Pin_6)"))
 (segment (start 89.735821 139.084179) (end 89.66 139.16) (width 0.6) (layer "B.Cu") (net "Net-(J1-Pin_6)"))
 (segment (start 89.735821 134.4) (end 89.735821 139.084179) (width 0.6) (layer "B.Cu") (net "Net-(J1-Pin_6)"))
 (via (at 97.2875 135.225) (size 0.6) (drill 0.3) (layers "F.Cu" "B.Cu") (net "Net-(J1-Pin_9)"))
 (segment (start 97.28 135.2325) (end 97.2875 135.225) (width 0.6) (layer "B.Cu") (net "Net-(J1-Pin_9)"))
 (segment (start 97.28 139.16) (end 97.28 135.2325) (width 0.6) (layer "B.Cu") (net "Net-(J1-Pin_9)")))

